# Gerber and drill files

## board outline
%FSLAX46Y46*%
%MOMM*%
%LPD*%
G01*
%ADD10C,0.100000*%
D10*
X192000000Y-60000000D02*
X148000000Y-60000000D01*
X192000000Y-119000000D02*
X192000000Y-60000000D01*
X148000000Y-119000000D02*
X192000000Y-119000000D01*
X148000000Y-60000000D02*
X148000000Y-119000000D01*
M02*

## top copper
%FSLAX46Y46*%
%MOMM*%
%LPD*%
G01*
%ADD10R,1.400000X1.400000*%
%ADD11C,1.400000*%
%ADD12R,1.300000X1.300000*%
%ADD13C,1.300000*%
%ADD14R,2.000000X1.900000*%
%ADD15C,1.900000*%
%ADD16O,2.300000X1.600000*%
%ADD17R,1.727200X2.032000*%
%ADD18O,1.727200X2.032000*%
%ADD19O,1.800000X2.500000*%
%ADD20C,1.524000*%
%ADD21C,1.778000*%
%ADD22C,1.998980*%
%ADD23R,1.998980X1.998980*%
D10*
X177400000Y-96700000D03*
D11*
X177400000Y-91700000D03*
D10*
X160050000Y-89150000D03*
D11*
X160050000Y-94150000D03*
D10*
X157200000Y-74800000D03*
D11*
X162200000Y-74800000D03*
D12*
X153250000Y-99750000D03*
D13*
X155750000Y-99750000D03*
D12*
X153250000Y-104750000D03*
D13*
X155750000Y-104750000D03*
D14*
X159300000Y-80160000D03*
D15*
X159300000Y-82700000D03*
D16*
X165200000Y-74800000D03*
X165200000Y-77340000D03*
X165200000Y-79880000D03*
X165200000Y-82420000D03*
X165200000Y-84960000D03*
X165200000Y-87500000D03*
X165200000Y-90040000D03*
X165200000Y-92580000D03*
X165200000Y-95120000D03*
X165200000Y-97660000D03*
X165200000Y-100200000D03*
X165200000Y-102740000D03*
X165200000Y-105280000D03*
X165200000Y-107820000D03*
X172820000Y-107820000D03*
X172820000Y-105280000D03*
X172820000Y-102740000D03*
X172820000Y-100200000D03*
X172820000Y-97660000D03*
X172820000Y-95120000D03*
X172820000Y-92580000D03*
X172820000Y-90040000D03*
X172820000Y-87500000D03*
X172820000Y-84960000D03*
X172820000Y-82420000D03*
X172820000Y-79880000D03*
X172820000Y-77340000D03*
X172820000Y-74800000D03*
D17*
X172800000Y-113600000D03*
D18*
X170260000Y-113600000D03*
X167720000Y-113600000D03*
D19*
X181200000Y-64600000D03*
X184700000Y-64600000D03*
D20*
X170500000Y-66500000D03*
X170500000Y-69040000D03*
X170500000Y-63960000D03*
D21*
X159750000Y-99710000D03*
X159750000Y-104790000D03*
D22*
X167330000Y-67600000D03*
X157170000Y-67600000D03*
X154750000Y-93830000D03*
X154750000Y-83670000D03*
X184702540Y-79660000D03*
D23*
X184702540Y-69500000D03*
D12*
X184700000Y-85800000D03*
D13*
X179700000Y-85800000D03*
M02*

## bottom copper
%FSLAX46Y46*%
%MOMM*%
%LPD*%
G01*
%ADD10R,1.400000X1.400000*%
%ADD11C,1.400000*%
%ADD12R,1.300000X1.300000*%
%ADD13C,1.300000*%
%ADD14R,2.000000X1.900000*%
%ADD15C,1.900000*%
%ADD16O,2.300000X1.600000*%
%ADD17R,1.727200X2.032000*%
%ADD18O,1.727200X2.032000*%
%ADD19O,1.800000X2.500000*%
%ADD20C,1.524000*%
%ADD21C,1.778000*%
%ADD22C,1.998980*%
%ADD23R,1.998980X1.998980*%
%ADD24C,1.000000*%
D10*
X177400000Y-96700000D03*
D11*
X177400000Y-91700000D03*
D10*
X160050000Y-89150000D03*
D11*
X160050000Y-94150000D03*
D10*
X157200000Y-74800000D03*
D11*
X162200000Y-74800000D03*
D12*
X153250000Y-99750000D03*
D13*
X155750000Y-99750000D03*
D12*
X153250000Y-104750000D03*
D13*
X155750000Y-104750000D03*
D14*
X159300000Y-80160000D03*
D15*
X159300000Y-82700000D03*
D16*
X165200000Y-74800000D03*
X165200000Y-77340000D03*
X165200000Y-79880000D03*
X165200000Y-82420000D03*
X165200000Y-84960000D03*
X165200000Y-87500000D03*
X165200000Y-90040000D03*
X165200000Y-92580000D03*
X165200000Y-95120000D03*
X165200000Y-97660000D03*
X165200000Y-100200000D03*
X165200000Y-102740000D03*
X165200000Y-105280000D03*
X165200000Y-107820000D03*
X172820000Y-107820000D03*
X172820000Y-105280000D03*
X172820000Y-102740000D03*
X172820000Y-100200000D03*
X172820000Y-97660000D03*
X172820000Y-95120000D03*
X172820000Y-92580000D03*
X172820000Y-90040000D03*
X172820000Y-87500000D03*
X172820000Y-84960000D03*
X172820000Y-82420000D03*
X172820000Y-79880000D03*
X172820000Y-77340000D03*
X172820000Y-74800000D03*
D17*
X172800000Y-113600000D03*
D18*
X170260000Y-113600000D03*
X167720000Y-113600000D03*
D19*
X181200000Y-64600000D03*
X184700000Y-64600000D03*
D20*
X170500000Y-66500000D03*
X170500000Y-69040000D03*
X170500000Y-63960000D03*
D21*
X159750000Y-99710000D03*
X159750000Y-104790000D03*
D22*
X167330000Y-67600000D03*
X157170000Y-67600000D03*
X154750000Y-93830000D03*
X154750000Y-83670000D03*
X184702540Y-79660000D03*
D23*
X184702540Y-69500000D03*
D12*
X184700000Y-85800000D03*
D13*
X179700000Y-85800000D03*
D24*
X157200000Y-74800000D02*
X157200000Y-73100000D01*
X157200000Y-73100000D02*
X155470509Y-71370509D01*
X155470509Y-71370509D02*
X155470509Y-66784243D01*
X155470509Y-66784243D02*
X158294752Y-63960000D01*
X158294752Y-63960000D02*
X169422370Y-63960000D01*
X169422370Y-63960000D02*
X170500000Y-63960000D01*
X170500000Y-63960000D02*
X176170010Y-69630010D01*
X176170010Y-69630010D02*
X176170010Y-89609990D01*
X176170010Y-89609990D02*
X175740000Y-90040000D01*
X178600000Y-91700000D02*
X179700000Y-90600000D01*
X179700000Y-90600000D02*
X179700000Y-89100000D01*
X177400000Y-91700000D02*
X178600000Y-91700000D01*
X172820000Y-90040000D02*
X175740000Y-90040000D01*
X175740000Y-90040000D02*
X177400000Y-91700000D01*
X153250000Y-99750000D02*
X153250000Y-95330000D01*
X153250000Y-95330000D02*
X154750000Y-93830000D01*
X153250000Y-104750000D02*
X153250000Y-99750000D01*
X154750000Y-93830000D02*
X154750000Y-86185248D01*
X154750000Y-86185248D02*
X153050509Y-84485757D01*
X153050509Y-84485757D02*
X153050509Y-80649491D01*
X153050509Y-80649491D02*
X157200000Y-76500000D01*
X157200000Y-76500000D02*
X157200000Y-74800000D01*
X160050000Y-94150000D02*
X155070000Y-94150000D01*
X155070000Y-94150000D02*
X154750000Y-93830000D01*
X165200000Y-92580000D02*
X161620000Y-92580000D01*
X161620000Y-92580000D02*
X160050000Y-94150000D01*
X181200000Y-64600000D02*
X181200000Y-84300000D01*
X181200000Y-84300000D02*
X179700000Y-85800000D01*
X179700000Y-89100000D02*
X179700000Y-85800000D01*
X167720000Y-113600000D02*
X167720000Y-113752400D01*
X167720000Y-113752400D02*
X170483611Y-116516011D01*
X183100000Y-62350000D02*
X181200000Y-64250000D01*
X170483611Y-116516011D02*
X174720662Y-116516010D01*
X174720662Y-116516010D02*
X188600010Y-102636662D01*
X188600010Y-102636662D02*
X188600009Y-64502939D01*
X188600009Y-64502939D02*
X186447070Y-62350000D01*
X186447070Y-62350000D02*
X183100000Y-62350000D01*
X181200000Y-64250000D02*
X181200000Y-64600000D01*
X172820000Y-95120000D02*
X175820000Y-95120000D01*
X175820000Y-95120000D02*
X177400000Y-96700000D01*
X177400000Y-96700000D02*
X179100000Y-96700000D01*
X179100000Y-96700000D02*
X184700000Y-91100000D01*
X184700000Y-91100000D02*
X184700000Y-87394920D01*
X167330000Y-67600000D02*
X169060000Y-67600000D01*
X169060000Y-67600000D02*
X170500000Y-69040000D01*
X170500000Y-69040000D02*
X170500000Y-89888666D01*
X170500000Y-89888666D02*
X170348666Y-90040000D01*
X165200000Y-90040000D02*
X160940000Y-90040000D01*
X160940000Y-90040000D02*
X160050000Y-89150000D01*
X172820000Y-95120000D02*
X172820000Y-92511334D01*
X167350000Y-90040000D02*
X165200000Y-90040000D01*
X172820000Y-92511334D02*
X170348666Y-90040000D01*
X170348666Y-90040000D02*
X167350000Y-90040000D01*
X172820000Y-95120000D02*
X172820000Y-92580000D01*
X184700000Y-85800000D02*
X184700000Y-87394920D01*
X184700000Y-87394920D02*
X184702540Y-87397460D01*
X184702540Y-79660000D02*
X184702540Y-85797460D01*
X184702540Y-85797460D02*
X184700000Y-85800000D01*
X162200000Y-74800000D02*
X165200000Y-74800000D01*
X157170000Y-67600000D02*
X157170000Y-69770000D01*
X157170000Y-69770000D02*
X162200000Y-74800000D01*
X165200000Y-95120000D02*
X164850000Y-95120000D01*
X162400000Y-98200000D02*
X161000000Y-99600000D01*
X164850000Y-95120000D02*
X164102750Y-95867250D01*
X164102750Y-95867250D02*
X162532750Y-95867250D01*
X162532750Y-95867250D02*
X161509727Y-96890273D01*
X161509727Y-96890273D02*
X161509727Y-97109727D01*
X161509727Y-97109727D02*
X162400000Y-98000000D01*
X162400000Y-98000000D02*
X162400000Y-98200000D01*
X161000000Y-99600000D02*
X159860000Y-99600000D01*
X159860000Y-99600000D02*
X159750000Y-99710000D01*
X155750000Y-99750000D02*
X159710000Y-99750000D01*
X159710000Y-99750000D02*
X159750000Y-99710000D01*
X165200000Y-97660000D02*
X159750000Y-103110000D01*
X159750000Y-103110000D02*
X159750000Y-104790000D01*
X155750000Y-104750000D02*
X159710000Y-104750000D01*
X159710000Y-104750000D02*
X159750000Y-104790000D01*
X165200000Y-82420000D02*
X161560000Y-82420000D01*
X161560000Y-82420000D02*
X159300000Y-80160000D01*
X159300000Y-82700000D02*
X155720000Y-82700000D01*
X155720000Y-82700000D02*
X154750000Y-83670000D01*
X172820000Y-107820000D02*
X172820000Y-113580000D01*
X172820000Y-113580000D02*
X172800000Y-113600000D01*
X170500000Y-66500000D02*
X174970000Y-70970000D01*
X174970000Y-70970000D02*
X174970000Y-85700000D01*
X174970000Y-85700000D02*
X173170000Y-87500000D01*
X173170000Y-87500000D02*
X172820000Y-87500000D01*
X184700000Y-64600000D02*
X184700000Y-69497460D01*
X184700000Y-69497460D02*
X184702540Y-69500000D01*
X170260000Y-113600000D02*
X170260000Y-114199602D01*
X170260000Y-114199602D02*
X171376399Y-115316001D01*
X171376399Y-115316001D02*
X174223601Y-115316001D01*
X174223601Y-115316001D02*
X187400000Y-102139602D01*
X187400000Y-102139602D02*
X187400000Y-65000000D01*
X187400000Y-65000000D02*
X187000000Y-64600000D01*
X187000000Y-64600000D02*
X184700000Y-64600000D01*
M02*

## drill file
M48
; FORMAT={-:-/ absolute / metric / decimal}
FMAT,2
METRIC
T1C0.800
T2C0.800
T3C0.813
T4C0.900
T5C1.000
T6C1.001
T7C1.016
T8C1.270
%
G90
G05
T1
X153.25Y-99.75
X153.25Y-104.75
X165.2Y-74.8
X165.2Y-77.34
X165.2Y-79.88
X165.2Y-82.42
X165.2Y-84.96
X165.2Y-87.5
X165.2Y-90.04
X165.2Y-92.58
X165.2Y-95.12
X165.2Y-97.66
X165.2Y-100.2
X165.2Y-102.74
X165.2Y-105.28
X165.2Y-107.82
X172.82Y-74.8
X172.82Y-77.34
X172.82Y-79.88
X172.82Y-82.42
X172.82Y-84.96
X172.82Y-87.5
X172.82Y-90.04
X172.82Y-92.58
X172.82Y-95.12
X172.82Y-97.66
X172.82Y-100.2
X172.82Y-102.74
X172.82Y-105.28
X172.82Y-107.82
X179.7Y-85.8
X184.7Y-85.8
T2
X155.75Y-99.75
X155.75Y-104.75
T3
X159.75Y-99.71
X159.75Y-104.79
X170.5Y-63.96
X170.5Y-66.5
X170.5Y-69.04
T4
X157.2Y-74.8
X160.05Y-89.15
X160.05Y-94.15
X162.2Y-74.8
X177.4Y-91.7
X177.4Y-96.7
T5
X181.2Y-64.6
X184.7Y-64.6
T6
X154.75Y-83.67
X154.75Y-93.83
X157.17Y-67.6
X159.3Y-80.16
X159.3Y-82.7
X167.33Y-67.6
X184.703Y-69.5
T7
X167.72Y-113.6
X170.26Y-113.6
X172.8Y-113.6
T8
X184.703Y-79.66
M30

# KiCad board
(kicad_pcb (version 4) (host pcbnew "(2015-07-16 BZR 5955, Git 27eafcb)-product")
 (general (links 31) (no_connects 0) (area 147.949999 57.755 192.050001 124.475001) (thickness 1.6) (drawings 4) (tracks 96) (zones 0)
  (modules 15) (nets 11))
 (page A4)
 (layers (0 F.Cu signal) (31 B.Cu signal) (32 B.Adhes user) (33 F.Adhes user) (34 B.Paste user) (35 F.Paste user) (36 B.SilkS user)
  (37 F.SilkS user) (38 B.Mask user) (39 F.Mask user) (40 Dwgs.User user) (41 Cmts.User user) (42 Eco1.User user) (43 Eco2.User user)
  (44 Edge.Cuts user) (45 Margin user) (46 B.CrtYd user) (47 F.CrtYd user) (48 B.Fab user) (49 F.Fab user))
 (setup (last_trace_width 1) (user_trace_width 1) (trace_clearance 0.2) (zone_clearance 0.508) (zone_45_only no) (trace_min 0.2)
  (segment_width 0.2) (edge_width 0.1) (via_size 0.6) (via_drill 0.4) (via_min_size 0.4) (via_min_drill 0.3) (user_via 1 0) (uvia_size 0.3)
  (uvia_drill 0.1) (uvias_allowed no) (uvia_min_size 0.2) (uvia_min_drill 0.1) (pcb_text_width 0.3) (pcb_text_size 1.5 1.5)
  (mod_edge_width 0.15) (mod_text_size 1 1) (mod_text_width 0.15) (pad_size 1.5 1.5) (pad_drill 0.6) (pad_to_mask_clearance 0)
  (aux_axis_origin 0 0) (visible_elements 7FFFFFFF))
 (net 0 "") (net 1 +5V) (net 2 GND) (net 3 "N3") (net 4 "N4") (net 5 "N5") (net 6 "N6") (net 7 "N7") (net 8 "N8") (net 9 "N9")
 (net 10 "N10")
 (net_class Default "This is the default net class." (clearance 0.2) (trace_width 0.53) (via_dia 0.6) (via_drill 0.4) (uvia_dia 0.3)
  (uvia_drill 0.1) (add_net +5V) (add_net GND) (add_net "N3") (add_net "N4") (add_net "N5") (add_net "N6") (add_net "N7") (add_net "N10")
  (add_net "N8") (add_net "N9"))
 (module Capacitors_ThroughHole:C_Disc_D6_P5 (layer F.Cu) (at 177.4 96.7 90)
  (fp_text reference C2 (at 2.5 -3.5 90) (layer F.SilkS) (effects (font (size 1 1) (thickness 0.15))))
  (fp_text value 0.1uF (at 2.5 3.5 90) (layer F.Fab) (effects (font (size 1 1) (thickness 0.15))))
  (pad 1 thru_hole rect (at 0 0 90) (size 1.4 1.4) (drill 0.9) (layers *.Cu *.Mask F.SilkS) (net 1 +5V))
  (pad 2 thru_hole circle (at 5 0 90) (size 1.4 1.4) (drill 0.9) (layers *.Cu *.Mask F.SilkS) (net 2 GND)))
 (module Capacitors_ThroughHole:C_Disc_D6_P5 (layer F.Cu) (at 160.05 89.15 270)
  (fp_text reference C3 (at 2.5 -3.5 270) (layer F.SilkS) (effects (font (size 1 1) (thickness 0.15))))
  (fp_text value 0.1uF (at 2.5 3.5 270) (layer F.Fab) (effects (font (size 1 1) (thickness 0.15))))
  (pad 1 thru_hole rect (at 0 0 270) (size 1.4 1.4) (drill 0.9) (layers *.Cu *.Mask F.SilkS) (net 1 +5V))
  (pad 2 thru_hole circle (at 5 0 270) (size 1.4 1.4) (drill 0.9) (layers *.Cu *.Mask F.SilkS) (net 2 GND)))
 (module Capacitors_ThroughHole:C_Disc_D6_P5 (layer F.Cu) (at 157.2 74.8)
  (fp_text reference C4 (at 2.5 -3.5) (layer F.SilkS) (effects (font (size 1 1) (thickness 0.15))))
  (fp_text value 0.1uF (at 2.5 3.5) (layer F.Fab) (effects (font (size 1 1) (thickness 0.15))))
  (pad 1 thru_hole rect (at 0 0) (size 1.4 1.4) (drill 0.9) (layers *.Cu *.Mask F.SilkS) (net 2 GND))
  (pad 2 thru_hole circle (at 5 0) (size 1.4 1.4) (drill 0.9) (layers *.Cu *.Mask F.SilkS) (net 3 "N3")))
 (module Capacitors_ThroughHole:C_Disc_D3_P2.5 (layer F.Cu) (at 153.25 99.75)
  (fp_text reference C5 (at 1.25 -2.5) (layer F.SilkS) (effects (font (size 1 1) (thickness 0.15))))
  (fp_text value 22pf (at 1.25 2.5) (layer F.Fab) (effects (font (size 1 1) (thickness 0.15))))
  (pad 1 thru_hole rect (at 0 0) (size 1.3 1.3) (drill 0.8) (layers *.Cu *.Mask F.SilkS) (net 2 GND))
  (pad 2 thru_hole circle (at 2.5 0) (size 1.3 1.3) (drill 0.8001) (layers *.Cu *.Mask F.SilkS) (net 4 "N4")))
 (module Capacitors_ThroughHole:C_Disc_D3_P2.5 (layer F.Cu) (at 153.25 104.75)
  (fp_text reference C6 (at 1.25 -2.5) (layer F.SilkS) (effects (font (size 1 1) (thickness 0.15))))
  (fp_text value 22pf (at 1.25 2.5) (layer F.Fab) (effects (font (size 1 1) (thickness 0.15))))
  (pad 1 thru_hole rect (at 0 0) (size 1.3 1.3) (drill 0.8) (layers *.Cu *.Mask F.SilkS) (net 2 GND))
  (pad 2 thru_hole circle (at 2.5 0) (size 1.3 1.3) (drill 0.8001) (layers *.Cu *.Mask F.SilkS) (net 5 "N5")))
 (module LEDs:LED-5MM (layer F.Cu) (at 159.3 80.16 270)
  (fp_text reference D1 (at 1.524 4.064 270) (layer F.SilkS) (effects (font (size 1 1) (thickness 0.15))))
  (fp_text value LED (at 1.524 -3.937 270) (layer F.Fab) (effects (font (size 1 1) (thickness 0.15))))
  (pad 1 thru_hole rect (at 0 0) (size 2 1.9) (drill 1.00076) (layers *.Cu *.Mask F.SilkS) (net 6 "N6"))
  (pad 2 thru_hole circle (at 2.54 0 270) (size 1.9 1.9) (drill 1.00076) (layers *.Cu *.Mask F.SilkS) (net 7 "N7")))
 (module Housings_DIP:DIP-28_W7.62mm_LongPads (layer F.Cu) (at 165.2 74.8)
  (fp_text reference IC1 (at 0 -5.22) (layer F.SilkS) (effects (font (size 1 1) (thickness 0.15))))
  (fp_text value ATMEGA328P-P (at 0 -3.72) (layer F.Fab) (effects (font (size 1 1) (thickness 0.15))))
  (pad 1 thru_hole oval (at 0 0) (size 2.3 1.6) (drill 0.8) (layers *.Cu *.Mask F.SilkS) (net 3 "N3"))
  (pad 2 thru_hole oval (at 0 2.54) (size 2.3 1.6) (drill 0.8) (layers *.Cu *.Mask F.SilkS))
  (pad 3 thru_hole oval (at 0 5.08) (size 2.3 1.6) (drill 0.8) (layers *.Cu *.Mask F.SilkS))
  (pad 4 thru_hole oval (at 0 7.62) (size 2.3 1.6) (drill 0.8) (layers *.Cu *.Mask F.SilkS) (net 6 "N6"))
  (pad 5 thru_hole oval (at 0 10.16) (size 2.3 1.6) (drill 0.8) (layers *.Cu *.Mask F.SilkS))
  (pad 6 thru_hole oval (at 0 12.7) (size 2.3 1.6) (drill 0.8) (layers *.Cu *.Mask F.SilkS))
  (pad 7 thru_hole oval (at 0 15.24) (size 2.3 1.6) (drill 0.8) (layers *.Cu *.Mask F.SilkS) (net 1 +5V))
  (pad 8 thru_hole oval (at 0 17.78) (size 2.3 1.6) (drill 0.8) (layers *.Cu *.Mask F.SilkS) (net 2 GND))
  (pad 9 thru_hole oval (at 0 20.32) (size 2.3 1.6) (drill 0.8) (layers *.Cu *.Mask F.SilkS) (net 4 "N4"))
  (pad 10 thru_hole oval (at 0 22.86) (size 2.3 1.6) (drill 0.8) (layers *.Cu *.Mask F.SilkS) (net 5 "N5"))
  (pad 11 thru_hole oval (at 0 25.4) (size 2.3 1.6) (drill 0.8) (layers *.Cu *.Mask F.SilkS))
  (pad 12 thru_hole oval (at 0 27.94) (size 2.3 1.6) (drill 0.8) (layers *.Cu *.Mask F.SilkS))
  (pad 13 thru_hole oval (at 0 30.48) (size 2.3 1.6) (drill 0.8) (layers *.Cu *.Mask F.SilkS))
  (pad 14 thru_hole oval (at 0 33.02) (size 2.3 1.6) (drill 0.8) (layers *.Cu *.Mask F.SilkS))
  (pad 15 thru_hole oval (at 7.62 33.02) (size 2.3 1.6) (drill 0.8) (layers *.Cu *.Mask F.SilkS) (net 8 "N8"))
  (pad 16 thru_hole oval (at 7.62 30.48) (size 2.3 1.6) (drill 0.8) (layers *.Cu *.Mask F.SilkS))
  (pad 17 thru_hole oval (at 7.62 27.94) (size 2.3 1.6) (drill 0.8) (layers *.Cu *.Mask F.SilkS))
  (pad 18 thru_hole oval (at 7.62 25.4) (size 2.3 1.6) (drill 0.8) (layers *.Cu *.Mask F.SilkS))
  (pad 19 thru_hole oval (at 7.62 22.86) (size 2.3 1.6) (drill 0.8) (layers *.Cu *.Mask F.SilkS))
  (pad 20 thru_hole oval (at 7.62 20.32) (size 2.3 1.6) (drill 0.8) (layers *.Cu *.Mask F.SilkS) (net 1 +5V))
  (pad 21 thru_hole oval (at 7.62 17.78) (size 2.3 1.6) (drill 0.8) (layers *.Cu *.Mask F.SilkS) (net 1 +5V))
  (pad 22 thru_hole oval (at 7.62 15.24) (size 2.3 1.6) (drill 0.8) (layers *.Cu *.Mask F.SilkS) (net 2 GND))
  (pad 23 thru_hole oval (at 7.62 12.7) (size 2.3 1.6) (drill 0.8) (layers *.Cu *.Mask F.SilkS) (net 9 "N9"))
  (pad 24 thru_hole oval (at 7.62 10.16) (size 2.3 1.6) (drill 0.8) (layers *.Cu *.Mask F.SilkS))
  (pad 25 thru_hole oval (at 7.62 7.62) (size 2.3 1.6) (drill 0.8) (layers *.Cu *.Mask F.SilkS))
  (pad 26 thru_hole oval (at 7.62 5.08) (size 2.3 1.6) (drill 0.8) (layers *.Cu *.Mask F.SilkS))
  (pad 27 thru_hole oval (at 7.62 2.54) (size 2.3 1.6) (drill 0.8) (layers *.Cu *.Mask F.SilkS))
  (pad 28 thru_hole oval (at 7.62 0) (size 2.3 1.6) (drill 0.8) (layers *.Cu *.Mask F.SilkS)))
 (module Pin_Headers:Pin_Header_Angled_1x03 (layer F.Cu) (at 172.8 113.6 270)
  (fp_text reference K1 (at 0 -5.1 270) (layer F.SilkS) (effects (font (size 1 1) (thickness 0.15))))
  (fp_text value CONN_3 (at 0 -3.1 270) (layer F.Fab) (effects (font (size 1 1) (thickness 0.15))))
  (pad 1 thru_hole rect (at 0 0 270) (size 2.032 1.7272) (drill 1.016) (layers *.Cu *.Mask F.SilkS) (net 8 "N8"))
  (pad 2 thru_hole oval (at 0 2.54 270) (size 2.032 1.7272) (drill 1.016) (layers *.Cu *.Mask F.SilkS) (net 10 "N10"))
  (pad 3 thru_hole oval (at 0 5.08 270) (size 2.032 1.7272) (drill 1.016) (layers *.Cu *.Mask F.SilkS) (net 2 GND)))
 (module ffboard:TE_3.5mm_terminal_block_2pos (layer F.Cu) (at 181.2 64.6)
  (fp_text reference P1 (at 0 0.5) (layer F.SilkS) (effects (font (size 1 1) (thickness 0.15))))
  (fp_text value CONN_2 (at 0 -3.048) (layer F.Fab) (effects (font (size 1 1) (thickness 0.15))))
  (pad 1 thru_hole oval (at 0 0) (size 1.8 2.5) (drill 1) (layers *.Cu *.Mask F.SilkS) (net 2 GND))
  (pad 2 thru_hole oval (at 3.5 0) (size 1.8 2.5) (drill 1) (layers *.Cu *.Mask F.SilkS) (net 10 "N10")))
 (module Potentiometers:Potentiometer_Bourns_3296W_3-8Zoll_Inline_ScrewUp (layer F.Cu) (at 170.5 63.96 180)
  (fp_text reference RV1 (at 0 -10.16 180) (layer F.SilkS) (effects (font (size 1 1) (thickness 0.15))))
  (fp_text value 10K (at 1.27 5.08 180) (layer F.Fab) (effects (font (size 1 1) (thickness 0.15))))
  (pad 2 thru_hole circle (at 0 -2.54 180) (size 1.524 1.524) (drill 0.8128) (layers *.Cu *.Mask F.SilkS) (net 9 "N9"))
  (pad 3 thru_hole circle (at 0 -5.08 180) (size 1.524 1.524) (drill 0.8128) (layers *.Cu *.Mask F.SilkS) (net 1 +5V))
  (pad 1 thru_hole circle (at 0 0 180) (size 1.524 1.524) (drill 0.8128) (layers *.Cu *.Mask F.SilkS) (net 2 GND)))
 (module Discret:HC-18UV (layer F.Cu) (at 159.75 102.25 270)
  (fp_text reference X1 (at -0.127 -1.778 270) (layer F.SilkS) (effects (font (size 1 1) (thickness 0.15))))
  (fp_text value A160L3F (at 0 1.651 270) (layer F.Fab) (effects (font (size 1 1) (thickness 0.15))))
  (pad 1 thru_hole circle (at -2.54 0 270) (size 1.778 1.778) (drill 0.8128) (layers *.Cu *.Mask F.SilkS) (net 4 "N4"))
  (pad 2 thru_hole circle (at 2.54 0 270) (size 1.778 1.778) (drill 0.8128) (layers *.Cu *.Mask F.SilkS) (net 5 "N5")))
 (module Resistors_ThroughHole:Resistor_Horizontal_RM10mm (layer F.Cu) (at 162.25 67.6 180)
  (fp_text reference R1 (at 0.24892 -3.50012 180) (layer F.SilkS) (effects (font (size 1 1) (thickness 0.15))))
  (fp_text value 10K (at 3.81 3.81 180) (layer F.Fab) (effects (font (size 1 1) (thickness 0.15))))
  (pad 1 thru_hole circle (at -5.08 0 180) (size 1.99898 1.99898) (drill 1.00076) (layers *.Cu *.SilkS *.Mask) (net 1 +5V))
  (pad 2 thru_hole circle (at 5.08 0 180) (size 1.99898 1.99898) (drill 1.00076) (layers *.Cu *.SilkS *.Mask) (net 3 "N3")))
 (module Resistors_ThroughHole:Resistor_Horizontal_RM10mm (layer F.Cu) (at 154.75 88.75 90)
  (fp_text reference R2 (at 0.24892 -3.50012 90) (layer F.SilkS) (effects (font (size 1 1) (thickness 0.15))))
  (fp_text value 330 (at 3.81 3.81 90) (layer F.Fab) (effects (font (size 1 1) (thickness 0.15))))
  (pad 1 thru_hole circle (at -5.08 0 90) (size 1.99898 1.99898) (drill 1.00076) (layers *.Cu *.SilkS *.Mask) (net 2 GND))
  (pad 2 thru_hole circle (at 5.08 0 90) (size 1.99898 1.99898) (drill 1.00076) (layers *.Cu *.SilkS *.Mask) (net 7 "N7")))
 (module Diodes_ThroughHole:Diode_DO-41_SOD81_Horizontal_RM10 (layer F.Cu) (at 184.7 69.5 270)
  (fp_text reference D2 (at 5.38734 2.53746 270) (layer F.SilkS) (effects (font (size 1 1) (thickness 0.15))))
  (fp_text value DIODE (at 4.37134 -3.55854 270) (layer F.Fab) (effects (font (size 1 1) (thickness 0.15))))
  (pad 2 thru_hole circle (at 10.16 -0.00254 90) (size 1.99898 1.99898) (drill 1.27) (layers *.Cu *.Mask F.SilkS) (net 1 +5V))
  (pad 1 thru_hole rect (at 0 -0.00254 90) (size 1.99898 1.99898) (drill 1.00076) (layers *.Cu *.Mask F.SilkS) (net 10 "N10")))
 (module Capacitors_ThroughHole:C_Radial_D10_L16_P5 (layer F.Cu) (at 184.7 85.8 180)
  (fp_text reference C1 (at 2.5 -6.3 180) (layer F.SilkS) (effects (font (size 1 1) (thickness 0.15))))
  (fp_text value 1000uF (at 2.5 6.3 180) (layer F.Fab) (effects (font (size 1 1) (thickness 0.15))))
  (pad 1 thru_hole rect (at 0 0 180) (size 1.3 1.3) (drill 0.8) (layers *.Cu *.Mask F.SilkS) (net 1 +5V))
  (pad 2 thru_hole circle (at 5 0 180) (size 1.3 1.3) (drill 0.8) (layers *.Cu *.Mask F.SilkS) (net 2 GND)))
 (gr_line (start 192 60) (end 148 60) (layer Edge.Cuts) (width 0.1))
 (gr_line (start 192 119) (end 192 60) (layer Edge.Cuts) (width 0.1))
 (gr_line (start 148 119) (end 192 119) (layer Edge.Cuts) (width 0.1))
 (gr_line (start 148 60) (end 148 119) (layer Edge.Cuts) (width 0.1))
 (segment (start 157.2 74.8) (end 157.2 73.1) (width 1) (layer B.Cu) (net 2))
 (segment (start 157.2 73.1) (end 155.470509 71.370509) (width 1) (layer B.Cu) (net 2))
 (segment (start 155.470509 71.370509) (end 155.470509 66.784243) (width 1) (layer B.Cu) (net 2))
 (segment (start 155.470509 66.784243) (end 158.294752 63.96) (width 1) (layer B.Cu) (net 2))
 (segment (start 158.294752 63.96) (end 169.42237 63.96) (width 1) (layer B.Cu) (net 2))
 (segment (start 169.42237 63.96) (end 170.5 63.96) (width 1) (layer B.Cu) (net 2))
 (segment (start 170.5 63.96) (end 176.17001 69.63001) (width 1) (layer B.Cu) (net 2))
 (segment (start 176.17001 69.63001) (end 176.17001 89.60999) (width 1) (layer B.Cu) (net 2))
 (segment (start 176.17001 89.60999) (end 175.74 90.04) (width 1) (layer B.Cu) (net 2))
 (segment (start 178.6 91.7) (end 179.7 90.6) (width 1) (layer B.Cu) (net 2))
 (segment (start 179.7 90.6) (end 179.7 89.1) (width 1) (layer B.Cu) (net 2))
 (segment (start 177.4 91.7) (end 178.6 91.7) (width 1) (layer B.Cu) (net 2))
 (segment (start 172.82 90.04) (end 175.74 90.04) (width 1) (layer B.Cu) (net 2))
 (segment (start 175.74 90.04) (end 177.4 91.7) (width 1) (layer B.Cu) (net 2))
 (segment (start 153.25 99.75) (end 153.25 95.33) (width 1) (layer B.Cu) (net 2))
 (segment (start 153.25 95.33) (end 154.75 93.83) (width 1) (layer B.Cu) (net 2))
 (segment (start 153.25 104.75) (end 153.25 99.75) (width 1) (layer B.Cu) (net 2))
 (segment (start 154.75 93.83) (end 154.75 86.185248) (width 1) (layer B.Cu) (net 2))
 (segment (start 154.75 86.185248) (end 153.050509 84.485757) (width 1) (layer B.Cu) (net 2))
 (segment (start 153.050509 84.485757) (end 153.050509 80.649491) (width 1) (layer B.Cu) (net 2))
 (segment (start 153.050509 80.649491) (end 157.2 76.5) (width 1) (layer B.Cu) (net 2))
 (segment (start 157.2 76.5) (end 157.2 74.8) (width 1) (layer B.Cu) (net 2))
 (segment (start 160.05 94.15) (end 155.07 94.15) (width 1) (layer B.Cu) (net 2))
 (segment (start 155.07 94.15) (end 154.75 93.83) (width 1) (layer B.Cu) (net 2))
 (segment (start 165.2 92.58) (end 161.62 92.58) (width 1) (layer B.Cu) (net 2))
 (segment (start 161.62 92.58) (end 160.05 94.15) (width 1) (layer B.Cu) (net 2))
 (segment (start 181.2 64.6) (end 181.2 84.3) (width 1) (layer B.Cu) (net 2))
 (segment (start 181.2 84.3) (end 179.7 85.8) (width 1) (layer B.Cu) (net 2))
 (segment (start 179.7 89.1) (end 179.7 85.8) (width 1) (layer B.Cu) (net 2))
 (segment (start 167.72 113.6) (end 167.72 113.7524) (width 1) (layer B.Cu) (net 2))
 (segment (start 167.72 113.7524) (end 170.483611 116.516011) (width 1) (layer B.Cu) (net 2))
 (segment (start 183.1 62.35) (end 181.2 64.25) (width 1) (layer B.Cu) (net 2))
 (segment (start 170.483611 116.516011) (end 174.720662 116.51601) (width 1) (layer B.Cu) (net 2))
 (segment (start 174.720662 116.51601) (end 188.60001 102.636662) (width 1) (layer B.Cu) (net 2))
 (segment (start 188.60001 102.636662) (end 188.600009 64.502939) (width 1) (layer B.Cu) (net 2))
 (segment (start 188.600009 64.502939) (end 186.44707 62.35) (width 1) (layer B.Cu) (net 2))
 (segment (start 186.44707 62.35) (end 183.1 62.35) (width 1) (layer B.Cu) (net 2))
 (segment (start 181.2 64.25) (end 181.2 64.6) (width 1) (layer B.Cu) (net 2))
 (segment (start 172.82 95.12) (end 175.82 95.12) (width 1) (layer B.Cu) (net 1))
 (segment (start 175.82 95.12) (end 177.4 96.7) (width 1) (layer B.Cu) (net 1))
 (segment (start 177.4 96.7) (end 179.1 96.7) (width 1) (layer B.Cu) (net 1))
 (segment (start 179.1 96.7) (end 184.7 91.1) (width 1) (layer B.Cu) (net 1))
 (segment (start 184.7 91.1) (end 184.7 87.39492) (width 1) (layer B.Cu) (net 1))
 (segment (start 167.33 67.6) (end 169.06 67.6) (width 1) (layer B.Cu) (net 1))
 (segment (start 169.06 67.6) (end 170.5 69.04) (width 1) (layer B.Cu) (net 1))
 (segment (start 170.5 69.04) (end 170.5 89.888666) (width 1) (layer B.Cu) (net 1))
 (segment (start 170.5 89.888666) (end 170.348666 90.04) (width 1) (layer B.Cu) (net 1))
 (segment (start 165.2 90.04) (end 160.94 90.04) (width 1) (layer B.Cu) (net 1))
 (segment (start 160.94 90.04) (end 160.05 89.15) (width 1) (layer B.Cu) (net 1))
 (segment (start 172.82 95.12) (end 172.82 92.511334) (width 1) (layer B.Cu) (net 1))
 (segment (start 167.35 90.04) (end 165.2 90.04) (width 1) (layer B.Cu) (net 1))
 (segment (start 172.82 92.511334) (end 170.348666 90.04) (width 1) (layer B.Cu) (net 1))
 (segment (start 170.348666 90.04) (end 167.35 90.04) (width 1) (layer B.Cu) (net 1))
 (segment (start 172.82 95.12) (end 172.82 92.58) (width 1) (layer B.Cu) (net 1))
 (segment (start 184.7 85.8) (end 184.7 87.39492) (width 1) (layer B.Cu) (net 1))
 (segment (start 184.7 87.39492) (end 184.70254 87.39746) (width 1) (layer B.Cu) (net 1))
 (segment (start 184.70254 79.66) (end 184.70254 85.79746) (width 1) (layer B.Cu) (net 1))
 (segment (start 184.70254 85.79746) (end 184.7 85.8) (width 1) (layer B.Cu) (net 1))
 (segment (start 162.2 74.8) (end 165.2 74.8) (width 1) (layer B.Cu) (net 3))
 (segment (start 157.17 67.6) (end 157.17 69.77) (width 1) (layer B.Cu) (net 3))
 (segment (start 157.17 69.77) (end 162.2 74.8) (width 1) (layer B.Cu) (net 3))
 (segment (start 165.2 95.12) (end 164.85 95.12) (width 1) (layer B.Cu) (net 4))
 (segment (start 162.4 98.2) (end 161 99.6) (width 1) (layer B.Cu) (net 4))
 (segment (start 164.85 95.12) (end 164.10275 95.86725) (width 1) (layer B.Cu) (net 4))
 (segment (start 164.10275 95.86725) (end 162.53275 95.86725) (width 1) (layer B.Cu) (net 4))
 (segment (start 162.53275 95.86725) (end 161.509727 96.890273) (width 1) (layer B.Cu) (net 4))
 (segment (start 161.509727 96.890273) (end 161.509727 97.109727) (width 1) (layer B.Cu) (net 4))
 (segment (start 161.509727 97.109727) (end 162.4 98) (width 1) (layer B.Cu) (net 4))
 (segment (start 162.4 98) (end 162.4 98.2) (width 1) (layer B.Cu) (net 4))
 (segment (start 161 99.6) (end 159.86 99.6) (width 1) (layer B.Cu) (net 4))
 (segment (start 159.86 99.6) (end 159.75 99.71) (width 1) (layer B.Cu) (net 4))
 (segment (start 155.75 99.75) (end 159.71 99.75) (width 1) (layer B.Cu) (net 4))
 (segment (start 159.71 99.75) (end 159.75 99.71) (width 1) (layer B.Cu) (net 4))
 (segment (start 165.2 97.66) (end 159.75 103.11) (width 1) (layer B.Cu) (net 5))
 (segment (start 159.75 103.11) (end 159.75 104.79) (width 1) (layer B.Cu) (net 5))
 (segment (start 155.75 104.75) (end 159.71 104.75) (width 1) (layer B.Cu) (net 5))
 (segment (start 159.71 104.75) (end 159.75 104.79) (width 1) (layer B.Cu) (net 5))
 (segment (start 165.2 82.42) (end 161.56 82.42) (width 1) (layer B.Cu) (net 6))
 (segment (start 161.56 82.42) (end 159.3 80.16) (width 1) (layer B.Cu) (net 6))
 (segment (start 159.3 82.7) (end 155.72 82.7) (width 1) (layer B.Cu) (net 7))
 (segment (start 155.72 82.7) (end 154.75 83.67) (width 1) (layer B.Cu) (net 7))
 (segment (start 172.82 107.82) (end 172.82 113.58) (width 1) (layer B.Cu) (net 8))
 (segment (start 172.82 113.58) (end 172.8 113.6) (width 1) (layer B.Cu) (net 8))
 (segment (start 170.5 66.5) (end 174.97 70.97) (width 1) (layer B.Cu) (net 9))
 (segment (start 174.97 70.97) (end 174.97 85.7) (width 1) (layer B.Cu) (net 9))
 (segment (start 174.97 85.7) (end 173.17 87.5) (width 1) (layer B.Cu) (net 9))
 (segment (start 173.17 87.5) (end 172.82 87.5) (width 1) (layer B.Cu) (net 9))
 (segment (start 184.7 64.6) (end 184.7 69.49746) (width 1) (layer B.Cu) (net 10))
 (segment (start 184.7 69.49746) (end 184.70254 69.5) (width 1) (layer B.Cu) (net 10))
 (segment (start 170.26 113.6) (end 170.26 114.199602) (width 1) (layer B.Cu) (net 10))
 (segment (start 170.26 114.199602) (end 171.376399 115.316001) (width 1) (layer B.Cu) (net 10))
 (segment (start 171.376399 115.316001) (end 174.223601 115.316001) (width 1) (layer B.Cu) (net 10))
 (segment (start 174.223601 115.316001) (end 187.4 102.139602) (width 1) (layer B.Cu) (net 10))
 (segment (start 187.4 102.139602) (end 187.4 65) (width 1) (layer B.Cu) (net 10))
 (segment (start 187.4 65) (end 187 64.6) (width 1) (layer B.Cu) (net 10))
 (segment (start 187 64.6) (end 184.7 64.6) (width 1) (layer B.Cu) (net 10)))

